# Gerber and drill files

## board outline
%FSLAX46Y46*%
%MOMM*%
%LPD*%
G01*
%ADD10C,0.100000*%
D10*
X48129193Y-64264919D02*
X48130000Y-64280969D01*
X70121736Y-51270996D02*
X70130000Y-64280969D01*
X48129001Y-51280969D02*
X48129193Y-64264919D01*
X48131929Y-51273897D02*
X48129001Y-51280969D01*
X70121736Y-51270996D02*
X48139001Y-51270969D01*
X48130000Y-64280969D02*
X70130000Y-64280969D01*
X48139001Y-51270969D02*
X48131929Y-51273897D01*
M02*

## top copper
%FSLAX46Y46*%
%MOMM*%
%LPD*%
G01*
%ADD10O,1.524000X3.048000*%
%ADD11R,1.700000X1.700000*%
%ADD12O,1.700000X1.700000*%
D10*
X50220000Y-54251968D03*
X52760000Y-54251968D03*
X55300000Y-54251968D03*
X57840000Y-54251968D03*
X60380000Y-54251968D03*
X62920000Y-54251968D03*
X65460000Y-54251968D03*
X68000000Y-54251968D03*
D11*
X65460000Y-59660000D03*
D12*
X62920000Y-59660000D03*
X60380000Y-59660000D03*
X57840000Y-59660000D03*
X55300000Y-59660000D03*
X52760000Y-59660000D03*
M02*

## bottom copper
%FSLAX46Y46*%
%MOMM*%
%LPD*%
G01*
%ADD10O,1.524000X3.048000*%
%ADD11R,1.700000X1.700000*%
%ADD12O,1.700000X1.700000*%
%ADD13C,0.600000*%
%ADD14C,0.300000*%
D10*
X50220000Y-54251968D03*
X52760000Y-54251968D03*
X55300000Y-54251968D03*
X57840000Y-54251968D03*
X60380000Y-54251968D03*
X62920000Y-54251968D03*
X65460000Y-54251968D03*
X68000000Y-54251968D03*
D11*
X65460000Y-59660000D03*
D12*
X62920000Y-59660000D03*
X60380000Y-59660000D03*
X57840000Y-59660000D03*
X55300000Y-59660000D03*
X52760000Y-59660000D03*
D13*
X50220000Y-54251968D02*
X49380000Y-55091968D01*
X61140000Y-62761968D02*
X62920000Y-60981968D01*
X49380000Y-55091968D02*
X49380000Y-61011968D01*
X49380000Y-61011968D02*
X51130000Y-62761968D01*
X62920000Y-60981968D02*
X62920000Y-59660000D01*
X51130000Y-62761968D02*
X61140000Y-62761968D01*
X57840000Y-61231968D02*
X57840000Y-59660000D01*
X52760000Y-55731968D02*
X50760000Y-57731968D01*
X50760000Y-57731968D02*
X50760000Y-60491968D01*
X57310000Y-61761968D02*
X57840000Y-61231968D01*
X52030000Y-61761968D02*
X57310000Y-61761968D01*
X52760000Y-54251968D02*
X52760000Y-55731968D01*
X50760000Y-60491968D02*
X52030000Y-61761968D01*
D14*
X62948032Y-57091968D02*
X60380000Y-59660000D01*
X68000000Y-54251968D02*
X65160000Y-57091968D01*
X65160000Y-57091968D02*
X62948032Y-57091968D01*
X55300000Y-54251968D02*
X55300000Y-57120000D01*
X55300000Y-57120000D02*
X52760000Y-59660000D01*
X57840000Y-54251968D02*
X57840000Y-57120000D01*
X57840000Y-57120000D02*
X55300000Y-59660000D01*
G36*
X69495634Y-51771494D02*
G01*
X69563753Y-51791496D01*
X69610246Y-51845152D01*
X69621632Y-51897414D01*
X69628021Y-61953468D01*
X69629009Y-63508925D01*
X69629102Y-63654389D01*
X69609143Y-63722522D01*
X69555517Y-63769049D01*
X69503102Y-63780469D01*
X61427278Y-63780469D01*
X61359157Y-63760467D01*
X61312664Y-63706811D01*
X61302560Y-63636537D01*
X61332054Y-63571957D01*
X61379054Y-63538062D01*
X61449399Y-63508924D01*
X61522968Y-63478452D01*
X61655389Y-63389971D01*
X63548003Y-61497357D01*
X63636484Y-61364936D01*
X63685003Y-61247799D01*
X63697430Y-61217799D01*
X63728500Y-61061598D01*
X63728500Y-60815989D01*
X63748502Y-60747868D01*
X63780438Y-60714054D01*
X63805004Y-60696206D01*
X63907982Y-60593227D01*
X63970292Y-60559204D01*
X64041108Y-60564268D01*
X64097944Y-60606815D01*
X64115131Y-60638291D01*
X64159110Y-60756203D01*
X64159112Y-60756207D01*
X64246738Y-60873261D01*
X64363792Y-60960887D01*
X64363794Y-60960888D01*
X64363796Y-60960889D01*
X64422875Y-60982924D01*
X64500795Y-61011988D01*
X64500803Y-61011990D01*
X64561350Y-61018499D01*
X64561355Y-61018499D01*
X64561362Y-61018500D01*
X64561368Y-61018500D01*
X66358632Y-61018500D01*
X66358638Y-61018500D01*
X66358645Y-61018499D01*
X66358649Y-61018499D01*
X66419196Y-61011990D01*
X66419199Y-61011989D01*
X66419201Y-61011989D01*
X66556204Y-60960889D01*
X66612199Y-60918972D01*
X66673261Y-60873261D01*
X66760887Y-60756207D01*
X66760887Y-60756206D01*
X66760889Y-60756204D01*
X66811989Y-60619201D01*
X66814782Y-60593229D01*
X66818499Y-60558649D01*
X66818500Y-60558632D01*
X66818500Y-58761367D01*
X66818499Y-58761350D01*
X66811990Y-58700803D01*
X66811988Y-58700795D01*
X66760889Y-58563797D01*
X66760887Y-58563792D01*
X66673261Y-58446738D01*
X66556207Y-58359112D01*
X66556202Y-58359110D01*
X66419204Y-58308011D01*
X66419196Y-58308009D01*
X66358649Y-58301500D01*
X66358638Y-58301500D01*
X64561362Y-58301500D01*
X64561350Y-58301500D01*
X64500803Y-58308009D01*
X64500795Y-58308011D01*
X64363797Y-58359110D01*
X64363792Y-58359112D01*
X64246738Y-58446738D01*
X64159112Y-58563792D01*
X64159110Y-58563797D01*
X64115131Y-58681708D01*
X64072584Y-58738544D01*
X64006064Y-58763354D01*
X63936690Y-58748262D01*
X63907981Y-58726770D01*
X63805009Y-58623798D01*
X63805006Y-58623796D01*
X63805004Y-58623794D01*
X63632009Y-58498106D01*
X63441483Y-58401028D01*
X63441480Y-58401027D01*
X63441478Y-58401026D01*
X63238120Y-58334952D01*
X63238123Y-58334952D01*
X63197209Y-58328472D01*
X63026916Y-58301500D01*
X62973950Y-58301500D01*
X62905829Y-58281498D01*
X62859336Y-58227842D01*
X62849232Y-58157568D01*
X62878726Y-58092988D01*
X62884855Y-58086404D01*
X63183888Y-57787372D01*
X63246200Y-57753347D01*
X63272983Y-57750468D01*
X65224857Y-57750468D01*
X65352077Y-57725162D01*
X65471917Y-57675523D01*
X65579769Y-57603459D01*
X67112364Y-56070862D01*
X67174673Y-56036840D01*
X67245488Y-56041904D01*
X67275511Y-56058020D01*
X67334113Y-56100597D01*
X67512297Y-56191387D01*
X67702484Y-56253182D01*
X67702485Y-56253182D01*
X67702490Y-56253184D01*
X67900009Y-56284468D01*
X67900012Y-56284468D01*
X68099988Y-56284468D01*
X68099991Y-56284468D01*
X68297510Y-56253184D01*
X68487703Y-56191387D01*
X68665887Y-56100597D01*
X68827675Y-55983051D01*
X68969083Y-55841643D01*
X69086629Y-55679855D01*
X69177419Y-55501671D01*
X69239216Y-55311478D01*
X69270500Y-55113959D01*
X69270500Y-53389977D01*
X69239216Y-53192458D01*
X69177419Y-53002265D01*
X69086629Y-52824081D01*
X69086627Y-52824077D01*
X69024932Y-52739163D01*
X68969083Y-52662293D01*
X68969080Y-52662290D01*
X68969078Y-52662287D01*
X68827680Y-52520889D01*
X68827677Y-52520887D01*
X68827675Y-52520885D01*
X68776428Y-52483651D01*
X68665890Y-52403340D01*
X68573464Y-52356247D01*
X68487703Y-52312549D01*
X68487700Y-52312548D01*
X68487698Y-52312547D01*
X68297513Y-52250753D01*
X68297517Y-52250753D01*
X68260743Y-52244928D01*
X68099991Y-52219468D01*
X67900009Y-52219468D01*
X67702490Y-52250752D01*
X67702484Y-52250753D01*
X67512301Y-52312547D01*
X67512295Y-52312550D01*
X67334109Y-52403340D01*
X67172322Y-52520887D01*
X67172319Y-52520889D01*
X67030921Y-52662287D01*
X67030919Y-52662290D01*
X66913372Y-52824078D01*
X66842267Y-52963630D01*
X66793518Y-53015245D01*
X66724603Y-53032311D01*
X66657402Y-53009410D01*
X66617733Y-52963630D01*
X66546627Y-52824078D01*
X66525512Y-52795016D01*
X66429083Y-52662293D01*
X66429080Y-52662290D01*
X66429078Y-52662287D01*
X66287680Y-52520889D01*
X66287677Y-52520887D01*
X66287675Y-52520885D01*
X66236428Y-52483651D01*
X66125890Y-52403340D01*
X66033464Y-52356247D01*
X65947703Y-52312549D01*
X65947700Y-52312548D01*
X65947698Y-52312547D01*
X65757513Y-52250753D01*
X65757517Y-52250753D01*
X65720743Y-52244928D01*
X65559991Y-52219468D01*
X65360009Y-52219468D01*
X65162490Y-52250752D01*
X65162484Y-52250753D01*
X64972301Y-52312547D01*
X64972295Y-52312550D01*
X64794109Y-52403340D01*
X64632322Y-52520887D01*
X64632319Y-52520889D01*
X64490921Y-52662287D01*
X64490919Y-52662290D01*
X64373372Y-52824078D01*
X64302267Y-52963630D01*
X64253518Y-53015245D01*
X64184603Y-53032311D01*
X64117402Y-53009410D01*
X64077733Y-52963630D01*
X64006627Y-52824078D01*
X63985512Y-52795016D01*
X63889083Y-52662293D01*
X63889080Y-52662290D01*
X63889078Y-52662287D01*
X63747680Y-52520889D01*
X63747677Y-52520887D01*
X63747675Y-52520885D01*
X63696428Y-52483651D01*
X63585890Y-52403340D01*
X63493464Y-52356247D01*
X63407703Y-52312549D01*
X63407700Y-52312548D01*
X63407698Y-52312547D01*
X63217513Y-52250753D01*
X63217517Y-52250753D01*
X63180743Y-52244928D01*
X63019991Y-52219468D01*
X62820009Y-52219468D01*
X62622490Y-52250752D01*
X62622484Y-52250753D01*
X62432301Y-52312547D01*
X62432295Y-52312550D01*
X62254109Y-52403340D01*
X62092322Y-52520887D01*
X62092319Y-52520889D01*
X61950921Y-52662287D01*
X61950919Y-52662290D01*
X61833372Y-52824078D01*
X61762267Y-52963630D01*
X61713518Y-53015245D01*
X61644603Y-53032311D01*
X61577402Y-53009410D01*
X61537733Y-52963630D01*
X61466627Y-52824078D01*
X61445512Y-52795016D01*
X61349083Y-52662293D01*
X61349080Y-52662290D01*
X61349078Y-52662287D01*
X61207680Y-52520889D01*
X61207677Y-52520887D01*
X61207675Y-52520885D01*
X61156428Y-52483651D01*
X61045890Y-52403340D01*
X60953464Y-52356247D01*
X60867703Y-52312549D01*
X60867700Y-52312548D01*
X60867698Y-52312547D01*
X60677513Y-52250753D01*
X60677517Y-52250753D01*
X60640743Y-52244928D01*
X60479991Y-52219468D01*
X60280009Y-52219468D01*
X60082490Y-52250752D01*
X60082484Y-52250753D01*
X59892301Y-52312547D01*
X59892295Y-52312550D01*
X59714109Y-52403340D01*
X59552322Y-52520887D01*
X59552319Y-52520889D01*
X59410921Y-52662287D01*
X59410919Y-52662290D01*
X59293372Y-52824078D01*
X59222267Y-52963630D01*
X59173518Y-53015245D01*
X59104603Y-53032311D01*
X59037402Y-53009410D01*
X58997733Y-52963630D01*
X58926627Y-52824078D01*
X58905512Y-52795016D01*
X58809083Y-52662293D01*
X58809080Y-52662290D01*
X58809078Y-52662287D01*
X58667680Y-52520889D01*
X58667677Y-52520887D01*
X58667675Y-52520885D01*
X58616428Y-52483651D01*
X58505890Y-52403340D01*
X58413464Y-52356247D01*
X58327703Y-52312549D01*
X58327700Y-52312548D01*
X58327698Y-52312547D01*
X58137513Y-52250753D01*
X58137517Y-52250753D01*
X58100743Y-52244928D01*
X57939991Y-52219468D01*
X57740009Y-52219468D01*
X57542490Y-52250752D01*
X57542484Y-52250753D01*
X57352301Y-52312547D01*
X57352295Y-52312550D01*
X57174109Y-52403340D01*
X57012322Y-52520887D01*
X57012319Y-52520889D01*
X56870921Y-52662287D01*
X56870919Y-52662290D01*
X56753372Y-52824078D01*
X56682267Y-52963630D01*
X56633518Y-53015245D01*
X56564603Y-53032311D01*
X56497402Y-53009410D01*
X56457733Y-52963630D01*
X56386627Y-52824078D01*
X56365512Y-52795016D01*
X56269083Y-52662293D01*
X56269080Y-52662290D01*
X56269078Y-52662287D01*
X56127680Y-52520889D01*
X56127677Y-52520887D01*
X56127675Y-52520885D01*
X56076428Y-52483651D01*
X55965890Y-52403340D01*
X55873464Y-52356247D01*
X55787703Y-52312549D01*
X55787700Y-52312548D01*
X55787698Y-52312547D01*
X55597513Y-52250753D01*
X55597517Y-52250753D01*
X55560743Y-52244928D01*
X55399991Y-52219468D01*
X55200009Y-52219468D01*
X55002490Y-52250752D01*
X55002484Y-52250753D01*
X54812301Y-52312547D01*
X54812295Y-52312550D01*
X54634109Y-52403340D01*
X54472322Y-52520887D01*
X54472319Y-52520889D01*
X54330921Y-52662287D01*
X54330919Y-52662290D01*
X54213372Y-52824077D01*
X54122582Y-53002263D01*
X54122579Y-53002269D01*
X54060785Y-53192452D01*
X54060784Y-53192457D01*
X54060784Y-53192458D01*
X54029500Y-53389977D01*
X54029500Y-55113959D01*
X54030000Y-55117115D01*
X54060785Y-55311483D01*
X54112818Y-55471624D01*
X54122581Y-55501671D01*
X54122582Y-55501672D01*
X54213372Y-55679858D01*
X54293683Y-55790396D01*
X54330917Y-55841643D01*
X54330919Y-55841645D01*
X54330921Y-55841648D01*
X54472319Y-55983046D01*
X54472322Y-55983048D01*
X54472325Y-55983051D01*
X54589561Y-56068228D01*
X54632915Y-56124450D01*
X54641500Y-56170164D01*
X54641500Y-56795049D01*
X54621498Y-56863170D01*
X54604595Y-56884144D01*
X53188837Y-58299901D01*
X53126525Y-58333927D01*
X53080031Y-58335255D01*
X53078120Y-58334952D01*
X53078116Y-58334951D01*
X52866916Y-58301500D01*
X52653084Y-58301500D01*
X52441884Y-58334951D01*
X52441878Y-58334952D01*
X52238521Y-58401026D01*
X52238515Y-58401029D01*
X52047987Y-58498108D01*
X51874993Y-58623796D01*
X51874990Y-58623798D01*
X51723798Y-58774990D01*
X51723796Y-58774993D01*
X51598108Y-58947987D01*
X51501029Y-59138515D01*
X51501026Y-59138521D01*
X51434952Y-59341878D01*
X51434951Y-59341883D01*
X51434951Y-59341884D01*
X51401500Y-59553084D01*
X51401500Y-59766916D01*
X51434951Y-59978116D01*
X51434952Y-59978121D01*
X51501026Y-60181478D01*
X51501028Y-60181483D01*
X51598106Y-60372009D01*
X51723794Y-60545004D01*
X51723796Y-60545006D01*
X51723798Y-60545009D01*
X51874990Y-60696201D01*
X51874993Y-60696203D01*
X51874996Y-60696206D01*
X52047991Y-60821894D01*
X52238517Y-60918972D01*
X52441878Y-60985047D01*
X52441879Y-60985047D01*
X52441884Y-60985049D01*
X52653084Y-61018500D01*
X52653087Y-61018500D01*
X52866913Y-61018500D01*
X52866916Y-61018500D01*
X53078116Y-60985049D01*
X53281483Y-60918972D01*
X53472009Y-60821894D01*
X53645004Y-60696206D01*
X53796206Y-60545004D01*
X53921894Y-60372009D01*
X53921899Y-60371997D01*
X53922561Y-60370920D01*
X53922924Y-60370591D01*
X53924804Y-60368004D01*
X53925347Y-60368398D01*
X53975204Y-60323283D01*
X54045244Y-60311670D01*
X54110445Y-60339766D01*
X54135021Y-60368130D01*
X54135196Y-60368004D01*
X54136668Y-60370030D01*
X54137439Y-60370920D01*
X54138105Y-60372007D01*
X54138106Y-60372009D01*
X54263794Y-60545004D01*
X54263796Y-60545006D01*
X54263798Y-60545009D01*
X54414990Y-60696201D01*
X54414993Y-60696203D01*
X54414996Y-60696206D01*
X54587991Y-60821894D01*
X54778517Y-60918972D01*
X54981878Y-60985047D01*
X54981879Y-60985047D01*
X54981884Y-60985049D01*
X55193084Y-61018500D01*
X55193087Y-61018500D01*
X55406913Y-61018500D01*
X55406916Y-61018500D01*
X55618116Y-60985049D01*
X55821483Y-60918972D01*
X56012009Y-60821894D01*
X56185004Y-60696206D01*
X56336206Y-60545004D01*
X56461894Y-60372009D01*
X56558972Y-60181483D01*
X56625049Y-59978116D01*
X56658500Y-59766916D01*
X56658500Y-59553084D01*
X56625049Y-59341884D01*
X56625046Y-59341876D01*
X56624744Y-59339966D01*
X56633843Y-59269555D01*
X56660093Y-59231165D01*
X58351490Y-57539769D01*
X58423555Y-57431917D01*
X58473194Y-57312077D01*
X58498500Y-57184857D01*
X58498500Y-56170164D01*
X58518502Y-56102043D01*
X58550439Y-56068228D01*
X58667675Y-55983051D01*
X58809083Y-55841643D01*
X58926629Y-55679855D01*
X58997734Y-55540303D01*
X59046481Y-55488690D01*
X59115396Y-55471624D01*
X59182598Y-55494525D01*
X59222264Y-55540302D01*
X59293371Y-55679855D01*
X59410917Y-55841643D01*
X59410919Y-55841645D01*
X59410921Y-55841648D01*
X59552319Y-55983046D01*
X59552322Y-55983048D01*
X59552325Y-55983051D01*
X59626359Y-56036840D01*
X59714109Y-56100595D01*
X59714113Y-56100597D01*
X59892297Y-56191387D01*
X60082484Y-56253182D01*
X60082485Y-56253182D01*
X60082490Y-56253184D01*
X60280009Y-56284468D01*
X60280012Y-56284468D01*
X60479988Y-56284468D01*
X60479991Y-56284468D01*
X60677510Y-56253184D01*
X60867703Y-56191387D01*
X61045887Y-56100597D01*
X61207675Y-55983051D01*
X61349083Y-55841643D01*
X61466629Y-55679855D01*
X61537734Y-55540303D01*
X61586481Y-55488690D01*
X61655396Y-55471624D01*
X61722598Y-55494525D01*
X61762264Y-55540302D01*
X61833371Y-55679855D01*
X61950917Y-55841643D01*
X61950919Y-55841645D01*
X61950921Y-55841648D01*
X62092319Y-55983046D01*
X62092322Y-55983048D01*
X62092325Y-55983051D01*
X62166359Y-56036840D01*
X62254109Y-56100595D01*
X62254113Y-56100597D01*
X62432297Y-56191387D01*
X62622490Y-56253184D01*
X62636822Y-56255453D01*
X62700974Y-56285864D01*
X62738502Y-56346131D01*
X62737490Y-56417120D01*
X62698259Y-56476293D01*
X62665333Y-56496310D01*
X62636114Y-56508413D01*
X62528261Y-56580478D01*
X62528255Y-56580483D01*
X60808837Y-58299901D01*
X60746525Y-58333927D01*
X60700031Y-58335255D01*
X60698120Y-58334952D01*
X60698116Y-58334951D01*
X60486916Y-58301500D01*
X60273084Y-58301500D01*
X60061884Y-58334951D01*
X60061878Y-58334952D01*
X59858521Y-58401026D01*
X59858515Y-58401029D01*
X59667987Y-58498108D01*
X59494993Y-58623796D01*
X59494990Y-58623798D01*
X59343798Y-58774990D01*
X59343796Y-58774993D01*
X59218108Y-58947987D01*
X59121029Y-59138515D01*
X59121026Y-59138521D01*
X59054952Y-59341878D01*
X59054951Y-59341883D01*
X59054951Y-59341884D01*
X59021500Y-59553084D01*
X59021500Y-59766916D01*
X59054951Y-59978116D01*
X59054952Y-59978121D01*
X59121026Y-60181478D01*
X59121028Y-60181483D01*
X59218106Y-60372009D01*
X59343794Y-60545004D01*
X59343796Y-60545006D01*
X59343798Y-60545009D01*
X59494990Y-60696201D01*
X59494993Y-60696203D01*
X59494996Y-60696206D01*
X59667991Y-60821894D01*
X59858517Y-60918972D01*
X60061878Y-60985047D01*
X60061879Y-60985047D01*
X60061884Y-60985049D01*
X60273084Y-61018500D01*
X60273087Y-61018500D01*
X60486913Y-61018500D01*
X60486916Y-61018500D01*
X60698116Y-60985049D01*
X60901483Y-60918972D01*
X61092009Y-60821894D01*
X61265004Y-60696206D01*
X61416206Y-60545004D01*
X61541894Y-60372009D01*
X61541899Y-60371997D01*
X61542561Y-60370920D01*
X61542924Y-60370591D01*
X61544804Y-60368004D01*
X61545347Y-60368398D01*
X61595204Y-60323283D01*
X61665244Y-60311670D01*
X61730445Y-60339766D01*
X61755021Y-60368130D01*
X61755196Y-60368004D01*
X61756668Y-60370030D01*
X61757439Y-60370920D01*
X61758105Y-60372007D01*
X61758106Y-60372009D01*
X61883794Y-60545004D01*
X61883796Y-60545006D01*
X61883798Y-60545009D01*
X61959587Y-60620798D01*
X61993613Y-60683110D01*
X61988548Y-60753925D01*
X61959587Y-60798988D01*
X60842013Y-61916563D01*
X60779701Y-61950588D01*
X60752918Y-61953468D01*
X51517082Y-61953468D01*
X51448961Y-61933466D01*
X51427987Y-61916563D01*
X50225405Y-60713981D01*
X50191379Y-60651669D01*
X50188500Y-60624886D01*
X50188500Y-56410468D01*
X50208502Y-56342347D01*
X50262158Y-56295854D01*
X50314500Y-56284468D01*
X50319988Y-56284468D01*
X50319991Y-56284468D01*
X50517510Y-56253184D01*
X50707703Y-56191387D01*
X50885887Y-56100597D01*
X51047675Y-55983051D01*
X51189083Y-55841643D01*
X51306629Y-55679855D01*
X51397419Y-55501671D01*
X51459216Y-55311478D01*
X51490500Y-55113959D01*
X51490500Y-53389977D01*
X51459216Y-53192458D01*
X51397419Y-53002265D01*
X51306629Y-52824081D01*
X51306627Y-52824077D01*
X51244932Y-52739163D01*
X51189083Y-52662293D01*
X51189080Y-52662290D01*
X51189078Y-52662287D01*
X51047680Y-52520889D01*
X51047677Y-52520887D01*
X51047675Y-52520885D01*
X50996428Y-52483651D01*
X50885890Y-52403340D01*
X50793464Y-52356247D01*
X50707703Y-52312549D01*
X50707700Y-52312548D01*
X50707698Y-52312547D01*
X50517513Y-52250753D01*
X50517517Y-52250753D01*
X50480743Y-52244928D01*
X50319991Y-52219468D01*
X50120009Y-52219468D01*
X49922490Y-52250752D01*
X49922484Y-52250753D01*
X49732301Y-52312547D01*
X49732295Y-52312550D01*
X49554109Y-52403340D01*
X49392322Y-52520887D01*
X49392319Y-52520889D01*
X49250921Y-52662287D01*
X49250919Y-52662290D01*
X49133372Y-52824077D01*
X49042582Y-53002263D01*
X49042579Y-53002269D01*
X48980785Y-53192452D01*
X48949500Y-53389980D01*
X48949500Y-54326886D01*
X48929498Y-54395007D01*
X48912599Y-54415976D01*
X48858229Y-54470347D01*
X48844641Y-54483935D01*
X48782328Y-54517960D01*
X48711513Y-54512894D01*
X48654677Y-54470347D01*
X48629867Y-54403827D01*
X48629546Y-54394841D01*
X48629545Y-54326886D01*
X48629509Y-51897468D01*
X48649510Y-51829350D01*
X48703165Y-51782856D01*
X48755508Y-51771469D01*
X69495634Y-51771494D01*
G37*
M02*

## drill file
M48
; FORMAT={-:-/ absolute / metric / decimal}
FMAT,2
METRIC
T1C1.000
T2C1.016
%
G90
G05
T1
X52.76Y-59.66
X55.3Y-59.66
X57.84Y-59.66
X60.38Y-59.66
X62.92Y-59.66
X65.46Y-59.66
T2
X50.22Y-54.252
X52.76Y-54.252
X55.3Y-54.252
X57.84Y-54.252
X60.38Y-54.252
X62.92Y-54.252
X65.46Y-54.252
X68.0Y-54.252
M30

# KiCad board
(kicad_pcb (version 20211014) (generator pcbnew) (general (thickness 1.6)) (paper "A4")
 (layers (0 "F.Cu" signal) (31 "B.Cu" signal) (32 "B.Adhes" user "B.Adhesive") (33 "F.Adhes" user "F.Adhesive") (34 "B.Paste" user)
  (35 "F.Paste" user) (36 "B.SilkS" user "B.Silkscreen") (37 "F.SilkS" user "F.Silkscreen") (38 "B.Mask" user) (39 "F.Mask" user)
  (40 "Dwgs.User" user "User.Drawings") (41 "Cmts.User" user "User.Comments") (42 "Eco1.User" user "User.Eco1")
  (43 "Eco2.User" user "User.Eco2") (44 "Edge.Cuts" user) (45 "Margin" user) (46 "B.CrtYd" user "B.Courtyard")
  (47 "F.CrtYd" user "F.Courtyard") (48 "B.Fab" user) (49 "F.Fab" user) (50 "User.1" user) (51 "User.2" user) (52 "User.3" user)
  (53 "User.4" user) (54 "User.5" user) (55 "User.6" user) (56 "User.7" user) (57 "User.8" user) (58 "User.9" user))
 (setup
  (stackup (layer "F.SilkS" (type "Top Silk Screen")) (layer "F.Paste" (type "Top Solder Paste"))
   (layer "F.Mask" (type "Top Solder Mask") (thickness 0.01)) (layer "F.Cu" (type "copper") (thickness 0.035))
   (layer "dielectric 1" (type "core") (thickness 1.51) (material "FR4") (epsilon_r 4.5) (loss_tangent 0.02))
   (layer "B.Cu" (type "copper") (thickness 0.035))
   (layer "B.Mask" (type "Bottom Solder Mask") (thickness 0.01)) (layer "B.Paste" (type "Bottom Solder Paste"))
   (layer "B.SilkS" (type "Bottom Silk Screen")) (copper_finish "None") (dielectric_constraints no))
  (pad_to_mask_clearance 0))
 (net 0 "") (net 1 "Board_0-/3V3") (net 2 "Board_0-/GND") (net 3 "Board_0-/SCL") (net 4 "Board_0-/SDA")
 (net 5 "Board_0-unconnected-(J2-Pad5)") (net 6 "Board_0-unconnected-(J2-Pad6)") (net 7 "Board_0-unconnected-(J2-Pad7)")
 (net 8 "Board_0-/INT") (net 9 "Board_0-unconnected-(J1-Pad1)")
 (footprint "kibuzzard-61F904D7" (layer "F.Cu") (at 69.22 60.371968 90)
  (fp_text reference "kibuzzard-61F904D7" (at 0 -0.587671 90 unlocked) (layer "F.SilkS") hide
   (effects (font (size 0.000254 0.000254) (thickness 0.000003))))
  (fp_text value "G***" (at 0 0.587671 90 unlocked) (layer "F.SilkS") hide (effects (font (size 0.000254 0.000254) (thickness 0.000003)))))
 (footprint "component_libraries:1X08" (layer "F.Cu") (at 59.11 54.251968)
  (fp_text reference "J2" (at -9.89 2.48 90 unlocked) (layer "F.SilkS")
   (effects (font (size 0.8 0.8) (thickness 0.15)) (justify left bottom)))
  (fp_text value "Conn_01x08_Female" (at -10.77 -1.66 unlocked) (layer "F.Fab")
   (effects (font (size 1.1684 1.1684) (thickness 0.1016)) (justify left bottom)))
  (pad "1" thru_hole oval (at -8.89 0 90) (size 3.048 1.524) (drill 1.016) (layers *.Cu *.Mask) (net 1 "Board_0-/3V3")
   (solder_mask_margin 0.1016))
  (pad "2" thru_hole oval (at -6.35 0 90) (size 3.048 1.524) (drill 1.016) (layers *.Cu *.Mask) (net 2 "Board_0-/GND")
   (solder_mask_margin 0.1016))
  (pad "3" thru_hole oval (at -3.81 0 90) (size 3.048 1.524) (drill 1.016) (layers *.Cu *.Mask) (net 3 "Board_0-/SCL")
   (solder_mask_margin 0.1016))
  (pad "4" thru_hole oval (at -1.27 0 90) (size 3.048 1.524) (drill 1.016) (layers *.Cu *.Mask) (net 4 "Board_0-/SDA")
   (solder_mask_margin 0.1016))
  (pad "5" thru_hole oval (at 1.27 0 90) (size 3.048 1.524) (drill 1.016) (layers *.Cu *.Mask) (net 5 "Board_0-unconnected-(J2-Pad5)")
   (solder_mask_margin 0.1016))
  (pad "6" thru_hole oval (at 3.81 0 90) (size 3.048 1.524) (drill 1.016) (layers *.Cu *.Mask) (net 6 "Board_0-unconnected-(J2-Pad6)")
   (solder_mask_margin 0.1016))
  (pad "7" thru_hole oval (at 6.35 0 90) (size 3.048 1.524) (drill 1.016) (layers *.Cu *.Mask) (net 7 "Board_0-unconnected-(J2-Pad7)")
   (solder_mask_margin 0.1016))
  (pad "8" thru_hole oval (at 8.89 0 90) (size 3.048 1.524) (drill 1.016) (layers *.Cu *.Mask) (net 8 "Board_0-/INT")
   (solder_mask_margin 0.1016)))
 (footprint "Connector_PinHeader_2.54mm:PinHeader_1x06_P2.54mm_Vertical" (layer "F.Cu") (at 65.46 59.66 -90)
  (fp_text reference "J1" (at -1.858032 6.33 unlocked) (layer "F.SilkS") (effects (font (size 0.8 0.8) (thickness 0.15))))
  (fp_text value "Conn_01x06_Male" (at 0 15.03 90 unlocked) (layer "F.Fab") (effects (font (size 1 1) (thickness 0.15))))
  (pad "1" thru_hole rect locked (at 0 0 270) (size 1.7 1.7) (drill 1) (layers *.Cu *.Mask) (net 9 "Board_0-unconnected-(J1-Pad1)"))
  (pad "2" thru_hole oval locked (at 0 2.54 270) (size 1.7 1.7) (drill 1) (layers *.Cu *.Mask) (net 1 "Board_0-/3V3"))
  (pad "3" thru_hole oval locked (at 0 5.08 270) (size 1.7 1.7) (drill 1) (layers *.Cu *.Mask) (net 8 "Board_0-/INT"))
  (pad "4" thru_hole oval locked (at 0 7.62 270) (size 1.7 1.7) (drill 1) (layers *.Cu *.Mask) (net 2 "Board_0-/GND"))
  (pad "5" thru_hole oval locked (at 0 10.16 270) (size 1.7 1.7) (drill 1) (layers *.Cu *.Mask) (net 4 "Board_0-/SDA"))
  (pad "6" thru_hole oval locked (at 0 12.7 270) (size 1.7 1.7) (drill 1) (layers *.Cu *.Mask) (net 3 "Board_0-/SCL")))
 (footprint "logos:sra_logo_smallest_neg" (layer "F.Cu") (at 49.26 59.581968 90)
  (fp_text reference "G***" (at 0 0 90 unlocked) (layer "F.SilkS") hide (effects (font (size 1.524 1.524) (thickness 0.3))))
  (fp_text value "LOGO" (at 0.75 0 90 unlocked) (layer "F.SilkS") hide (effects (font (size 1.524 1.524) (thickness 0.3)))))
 (gr_line (start 48.129193 64.264919) (end 48.13 64.280969) (layer "Edge.Cuts") (width 0.1))
 (gr_line (start 70.121736 51.270996) (end 70.13 64.280969) (layer "Edge.Cuts") (width 0.1))
 (gr_line (start 48.129001 51.280969) (end 48.129193 64.264919) (layer "Edge.Cuts") (width 0.1))
 (gr_line (start 48.131929 51.273897) (end 48.129001 51.280969) (layer "Edge.Cuts") (width 0.1))
 (gr_line (start 70.121736 51.270996) (end 48.139001 51.270969) (layer "Edge.Cuts") (width 0.1))
 (gr_line (start 48.13 64.280969) (end 70.13 64.280969) (layer "Edge.Cuts") (width 0.1))
 (gr_line (start 48.139001 51.270969) (end 48.131929 51.273897) (layer "Edge.Cuts") (width 0.1))
 (segment (start 50.22 54.251968) (end 49.38 55.091968) (width 0.6) (layer "B.Cu") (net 1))
 (segment (start 61.14 62.761968) (end 62.92 60.981968) (width 0.6) (layer "B.Cu") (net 1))
 (segment (start 49.38 55.091968) (end 49.38 61.011968) (width 0.6) (layer "B.Cu") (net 1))
 (segment (start 49.38 61.011968) (end 51.13 62.761968) (width 0.6) (layer "B.Cu") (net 1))
 (segment (start 62.92 60.981968) (end 62.92 59.66) (width 0.6) (layer "B.Cu") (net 1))
 (segment (start 51.13 62.761968) (end 61.14 62.761968) (width 0.6) (layer "B.Cu") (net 1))
 (segment (start 57.84 61.231968) (end 57.84 59.66) (width 0.6) (layer "B.Cu") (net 2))
 (segment (start 52.76 55.731968) (end 50.76 57.731968) (width 0.6) (layer "B.Cu") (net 2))
 (segment (start 50.76 57.731968) (end 50.76 60.491968) (width 0.6) (layer "B.Cu") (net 2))
 (segment (start 57.31 61.761968) (end 57.84 61.231968) (width 0.6) (layer "B.Cu") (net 2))
 (segment (start 52.03 61.761968) (end 57.31 61.761968) (width 0.6) (layer "B.Cu") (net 2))
 (segment (start 52.76 54.251968) (end 52.76 55.731968) (width 0.6) (layer "B.Cu") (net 2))
 (segment (start 50.76 60.491968) (end 52.03 61.761968) (width 0.6) (layer "B.Cu") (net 2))
 (segment (start 62.948032 57.091968) (end 60.38 59.66) (width 0.3) (layer "B.Cu") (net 8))
 (segment (start 68 54.251968) (end 65.16 57.091968) (width 0.3) (layer "B.Cu") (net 8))
 (segment (start 65.16 57.091968) (end 62.948032 57.091968) (width 0.3) (layer "B.Cu") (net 8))
 (segment (start 55.3 54.251968) (end 55.3 57.12) (width 0.3) (layer "B.Cu") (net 3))
 (segment (start 55.3 57.12) (end 52.76 59.66) (width 0.3) (layer "B.Cu") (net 3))
 (segment (start 57.84 54.251968) (end 57.84 57.12) (width 0.3) (layer "B.Cu") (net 4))
 (segment (start 57.84 57.12) (end 55.3 59.66) (width 0.3) (layer "B.Cu") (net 4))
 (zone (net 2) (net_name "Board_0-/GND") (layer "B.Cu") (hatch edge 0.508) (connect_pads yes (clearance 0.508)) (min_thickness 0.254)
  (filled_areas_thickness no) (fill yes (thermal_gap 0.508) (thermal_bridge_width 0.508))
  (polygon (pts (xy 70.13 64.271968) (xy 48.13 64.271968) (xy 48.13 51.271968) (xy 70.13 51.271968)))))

